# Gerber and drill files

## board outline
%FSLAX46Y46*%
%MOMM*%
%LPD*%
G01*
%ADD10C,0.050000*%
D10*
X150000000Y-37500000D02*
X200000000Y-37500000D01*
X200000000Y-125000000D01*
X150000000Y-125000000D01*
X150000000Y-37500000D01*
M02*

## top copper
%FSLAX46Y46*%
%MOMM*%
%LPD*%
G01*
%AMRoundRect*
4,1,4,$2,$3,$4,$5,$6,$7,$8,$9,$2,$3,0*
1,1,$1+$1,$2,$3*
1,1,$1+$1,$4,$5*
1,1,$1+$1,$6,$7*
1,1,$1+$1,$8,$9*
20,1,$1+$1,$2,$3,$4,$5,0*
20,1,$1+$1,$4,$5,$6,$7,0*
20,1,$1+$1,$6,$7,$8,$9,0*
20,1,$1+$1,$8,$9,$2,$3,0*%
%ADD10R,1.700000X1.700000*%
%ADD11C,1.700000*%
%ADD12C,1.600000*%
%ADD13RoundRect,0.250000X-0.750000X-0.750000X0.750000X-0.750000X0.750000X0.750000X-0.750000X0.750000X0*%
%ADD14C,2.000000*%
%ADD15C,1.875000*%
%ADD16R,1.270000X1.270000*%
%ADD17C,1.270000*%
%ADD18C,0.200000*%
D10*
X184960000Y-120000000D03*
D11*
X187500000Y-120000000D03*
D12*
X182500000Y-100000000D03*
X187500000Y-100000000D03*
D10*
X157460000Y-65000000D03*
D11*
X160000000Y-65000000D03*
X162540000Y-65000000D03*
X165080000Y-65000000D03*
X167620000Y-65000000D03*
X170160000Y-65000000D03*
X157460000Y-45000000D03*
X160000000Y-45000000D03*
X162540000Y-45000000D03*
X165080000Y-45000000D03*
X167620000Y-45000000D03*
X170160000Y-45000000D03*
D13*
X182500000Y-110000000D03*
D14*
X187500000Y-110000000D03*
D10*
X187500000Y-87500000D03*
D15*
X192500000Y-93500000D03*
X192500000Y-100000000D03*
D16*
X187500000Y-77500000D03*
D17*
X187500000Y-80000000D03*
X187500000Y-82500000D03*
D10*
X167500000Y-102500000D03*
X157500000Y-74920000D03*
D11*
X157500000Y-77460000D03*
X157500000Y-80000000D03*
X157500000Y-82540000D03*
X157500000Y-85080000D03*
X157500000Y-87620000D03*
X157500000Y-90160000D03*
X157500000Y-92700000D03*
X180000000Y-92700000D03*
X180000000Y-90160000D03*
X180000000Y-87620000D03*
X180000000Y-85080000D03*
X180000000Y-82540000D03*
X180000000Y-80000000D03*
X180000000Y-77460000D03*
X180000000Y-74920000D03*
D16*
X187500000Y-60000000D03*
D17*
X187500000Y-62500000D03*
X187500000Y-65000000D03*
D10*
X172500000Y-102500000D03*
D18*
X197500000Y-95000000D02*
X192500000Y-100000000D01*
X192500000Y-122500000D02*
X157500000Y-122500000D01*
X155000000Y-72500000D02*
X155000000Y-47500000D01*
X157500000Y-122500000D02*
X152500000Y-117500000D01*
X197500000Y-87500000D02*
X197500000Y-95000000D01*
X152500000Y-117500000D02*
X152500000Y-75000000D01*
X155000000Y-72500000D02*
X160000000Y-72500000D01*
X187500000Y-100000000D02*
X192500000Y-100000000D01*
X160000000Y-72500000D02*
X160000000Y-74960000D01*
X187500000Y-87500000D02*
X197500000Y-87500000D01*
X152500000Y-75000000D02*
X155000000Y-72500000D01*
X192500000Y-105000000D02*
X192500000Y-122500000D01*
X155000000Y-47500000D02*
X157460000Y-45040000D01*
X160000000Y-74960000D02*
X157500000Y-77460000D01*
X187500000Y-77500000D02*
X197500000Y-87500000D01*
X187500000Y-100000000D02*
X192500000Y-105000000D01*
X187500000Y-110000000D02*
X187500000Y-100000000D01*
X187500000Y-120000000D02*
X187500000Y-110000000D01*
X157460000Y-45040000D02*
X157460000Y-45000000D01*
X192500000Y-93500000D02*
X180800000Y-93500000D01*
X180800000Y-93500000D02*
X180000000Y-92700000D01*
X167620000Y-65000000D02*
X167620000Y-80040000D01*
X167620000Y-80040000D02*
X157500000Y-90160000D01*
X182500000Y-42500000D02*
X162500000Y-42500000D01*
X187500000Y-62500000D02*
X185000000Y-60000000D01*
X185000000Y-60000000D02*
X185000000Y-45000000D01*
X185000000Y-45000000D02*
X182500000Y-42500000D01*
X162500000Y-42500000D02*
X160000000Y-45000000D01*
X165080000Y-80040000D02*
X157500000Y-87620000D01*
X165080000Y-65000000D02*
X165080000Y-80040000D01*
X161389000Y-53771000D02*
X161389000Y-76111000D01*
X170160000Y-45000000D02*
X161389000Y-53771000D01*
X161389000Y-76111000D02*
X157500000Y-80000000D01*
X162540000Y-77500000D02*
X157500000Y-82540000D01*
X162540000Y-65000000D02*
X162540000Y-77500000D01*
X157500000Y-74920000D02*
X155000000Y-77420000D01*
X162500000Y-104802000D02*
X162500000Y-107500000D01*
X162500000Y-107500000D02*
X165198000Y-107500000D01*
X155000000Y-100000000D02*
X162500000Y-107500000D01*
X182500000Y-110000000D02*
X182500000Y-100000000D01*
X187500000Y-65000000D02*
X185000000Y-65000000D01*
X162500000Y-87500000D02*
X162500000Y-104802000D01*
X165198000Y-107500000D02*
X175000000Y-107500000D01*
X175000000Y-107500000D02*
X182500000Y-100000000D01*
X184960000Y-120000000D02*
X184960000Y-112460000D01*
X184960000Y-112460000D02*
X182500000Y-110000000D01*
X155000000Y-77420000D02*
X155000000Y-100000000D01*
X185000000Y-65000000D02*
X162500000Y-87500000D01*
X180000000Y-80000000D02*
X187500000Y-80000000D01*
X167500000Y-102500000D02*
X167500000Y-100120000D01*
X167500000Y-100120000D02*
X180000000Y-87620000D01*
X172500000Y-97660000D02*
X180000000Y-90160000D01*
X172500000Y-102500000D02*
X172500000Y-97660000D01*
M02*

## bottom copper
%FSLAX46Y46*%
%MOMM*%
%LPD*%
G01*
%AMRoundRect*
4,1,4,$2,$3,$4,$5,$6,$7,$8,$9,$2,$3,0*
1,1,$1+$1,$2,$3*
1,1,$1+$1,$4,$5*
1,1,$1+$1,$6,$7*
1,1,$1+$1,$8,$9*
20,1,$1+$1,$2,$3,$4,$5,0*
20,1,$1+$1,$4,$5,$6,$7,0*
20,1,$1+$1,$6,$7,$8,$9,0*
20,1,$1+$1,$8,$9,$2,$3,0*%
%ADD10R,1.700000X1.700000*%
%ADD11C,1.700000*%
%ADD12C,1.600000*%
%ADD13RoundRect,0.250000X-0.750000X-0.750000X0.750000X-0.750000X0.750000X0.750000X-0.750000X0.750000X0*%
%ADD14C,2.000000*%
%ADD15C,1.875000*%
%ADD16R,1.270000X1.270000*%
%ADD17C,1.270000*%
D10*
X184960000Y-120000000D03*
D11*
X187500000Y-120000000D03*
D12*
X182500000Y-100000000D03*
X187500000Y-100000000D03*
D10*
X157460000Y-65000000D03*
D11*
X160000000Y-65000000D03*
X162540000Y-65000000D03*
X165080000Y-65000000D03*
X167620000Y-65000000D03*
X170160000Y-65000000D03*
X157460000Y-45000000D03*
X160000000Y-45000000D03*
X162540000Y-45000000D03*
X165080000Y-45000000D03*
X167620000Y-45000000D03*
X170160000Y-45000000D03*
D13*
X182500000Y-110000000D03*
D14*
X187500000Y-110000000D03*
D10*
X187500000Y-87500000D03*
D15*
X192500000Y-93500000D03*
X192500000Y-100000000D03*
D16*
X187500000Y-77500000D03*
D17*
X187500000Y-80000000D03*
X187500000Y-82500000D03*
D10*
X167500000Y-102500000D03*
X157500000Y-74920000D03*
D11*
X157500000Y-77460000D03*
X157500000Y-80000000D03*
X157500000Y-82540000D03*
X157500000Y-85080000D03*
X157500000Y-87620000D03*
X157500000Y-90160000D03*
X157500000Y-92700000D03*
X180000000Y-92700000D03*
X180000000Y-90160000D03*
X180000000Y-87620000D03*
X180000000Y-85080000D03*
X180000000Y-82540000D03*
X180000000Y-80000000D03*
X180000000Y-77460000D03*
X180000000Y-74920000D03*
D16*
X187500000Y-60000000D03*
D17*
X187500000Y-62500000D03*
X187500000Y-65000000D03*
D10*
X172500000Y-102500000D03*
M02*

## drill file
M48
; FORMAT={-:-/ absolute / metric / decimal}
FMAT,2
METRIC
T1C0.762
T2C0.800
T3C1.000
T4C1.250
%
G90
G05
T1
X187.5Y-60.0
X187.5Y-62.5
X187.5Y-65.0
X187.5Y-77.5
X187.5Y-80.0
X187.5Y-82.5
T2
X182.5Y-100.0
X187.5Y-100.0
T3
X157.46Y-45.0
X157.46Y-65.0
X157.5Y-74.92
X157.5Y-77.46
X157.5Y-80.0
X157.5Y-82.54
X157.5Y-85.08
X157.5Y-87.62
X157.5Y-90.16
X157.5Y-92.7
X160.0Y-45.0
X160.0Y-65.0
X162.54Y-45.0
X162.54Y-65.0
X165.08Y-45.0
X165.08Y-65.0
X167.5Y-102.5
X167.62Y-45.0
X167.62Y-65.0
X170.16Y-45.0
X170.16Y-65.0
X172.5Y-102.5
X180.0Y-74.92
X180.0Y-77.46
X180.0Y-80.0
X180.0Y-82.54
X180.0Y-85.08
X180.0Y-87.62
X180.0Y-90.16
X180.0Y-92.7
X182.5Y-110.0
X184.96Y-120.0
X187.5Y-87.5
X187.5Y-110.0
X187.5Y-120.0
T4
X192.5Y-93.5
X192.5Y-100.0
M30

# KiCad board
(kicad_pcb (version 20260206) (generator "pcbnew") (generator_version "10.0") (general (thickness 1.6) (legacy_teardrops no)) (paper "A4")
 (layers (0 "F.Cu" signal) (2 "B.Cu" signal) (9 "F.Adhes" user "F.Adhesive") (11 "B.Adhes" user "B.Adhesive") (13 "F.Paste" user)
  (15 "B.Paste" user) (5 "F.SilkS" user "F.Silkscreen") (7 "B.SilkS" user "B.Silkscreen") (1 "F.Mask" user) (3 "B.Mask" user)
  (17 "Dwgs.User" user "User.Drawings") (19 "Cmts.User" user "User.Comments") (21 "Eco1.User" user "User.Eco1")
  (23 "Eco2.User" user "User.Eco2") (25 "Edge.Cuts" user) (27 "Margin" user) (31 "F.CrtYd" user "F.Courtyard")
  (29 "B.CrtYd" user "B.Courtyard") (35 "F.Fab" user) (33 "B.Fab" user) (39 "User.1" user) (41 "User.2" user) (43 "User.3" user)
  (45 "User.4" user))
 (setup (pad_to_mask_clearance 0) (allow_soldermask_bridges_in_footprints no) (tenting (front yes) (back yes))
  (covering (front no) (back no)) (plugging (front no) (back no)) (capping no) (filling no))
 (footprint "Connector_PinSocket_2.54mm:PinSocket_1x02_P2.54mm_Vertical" (layer "F.Cu") (at 184.96 120 90)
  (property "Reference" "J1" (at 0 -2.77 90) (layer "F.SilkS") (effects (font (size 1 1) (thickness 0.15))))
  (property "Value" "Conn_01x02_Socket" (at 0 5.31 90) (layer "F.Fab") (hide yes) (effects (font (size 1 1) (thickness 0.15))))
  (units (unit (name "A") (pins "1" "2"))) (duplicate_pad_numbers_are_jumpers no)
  (pad "1" thru_hole rect (at 0 0 90) (size 1.7 1.7) (drill 1) (layers "*.Cu" "*.Mask") (remove_unused_layers no) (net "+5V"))
  (pad "2" thru_hole circle (at 0 2.54 90) (size 1.7 1.7) (drill 1) (layers "*.Cu" "*.Mask") (remove_unused_layers no) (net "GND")))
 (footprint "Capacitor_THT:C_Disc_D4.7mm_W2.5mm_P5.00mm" (layer "F.Cu") (at 182.5 100)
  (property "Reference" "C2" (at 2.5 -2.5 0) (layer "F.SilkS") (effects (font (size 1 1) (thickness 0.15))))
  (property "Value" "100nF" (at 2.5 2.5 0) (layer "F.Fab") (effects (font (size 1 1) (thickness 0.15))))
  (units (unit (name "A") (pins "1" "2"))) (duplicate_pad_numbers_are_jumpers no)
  (pad "1" thru_hole circle (at 0 0) (size 1.6 1.6) (drill 0.8) (layers "*.Cu" "*.Mask") (remove_unused_layers no) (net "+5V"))
  (pad "2" thru_hole circle (at 5 0) (size 1.6 1.6) (drill 0.8) (layers "*.Cu" "*.Mask") (remove_unused_layers no) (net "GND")))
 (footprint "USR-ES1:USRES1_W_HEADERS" (layer "F.Cu") (at 163.69 55 90)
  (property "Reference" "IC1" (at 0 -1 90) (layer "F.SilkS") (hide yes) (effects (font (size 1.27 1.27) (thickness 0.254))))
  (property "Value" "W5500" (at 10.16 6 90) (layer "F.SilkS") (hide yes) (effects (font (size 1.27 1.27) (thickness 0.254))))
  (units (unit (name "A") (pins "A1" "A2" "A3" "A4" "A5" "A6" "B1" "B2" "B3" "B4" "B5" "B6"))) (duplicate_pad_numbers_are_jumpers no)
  (pad "A1" thru_hole rect (at -10 -6.23 90) (size 1.7 1.7) (drill 1) (layers "*.Cu" "*.Mask") (remove_unused_layers no)
   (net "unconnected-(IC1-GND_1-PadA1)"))
  (pad "A2" thru_hole circle (at -10 -3.69 90) (size 1.7 1.7) (drill 1) (layers "*.Cu" "*.Mask") (remove_unused_layers no)
   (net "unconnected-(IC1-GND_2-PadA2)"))
  (pad "A3" thru_hole circle (at -10 -1.15 90) (size 1.7 1.7) (drill 1) (layers "*.Cu" "*.Mask") (remove_unused_layers no)
   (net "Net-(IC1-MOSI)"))
  (pad "A4" thru_hole circle (at -10 1.39 90) (size 1.7 1.7) (drill 1) (layers "*.Cu" "*.Mask") (remove_unused_layers no)
   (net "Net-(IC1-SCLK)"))
  (pad "A5" thru_hole circle (at -10 3.93 90) (size 1.7 1.7) (drill 1) (layers "*.Cu" "*.Mask") (remove_unused_layers no)
   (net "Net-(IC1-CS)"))
  (pad "A6" thru_hole circle (at -10 6.47 90) (size 1.7 1.7) (drill 1) (layers "*.Cu" "*.Mask") (remove_unused_layers no)
   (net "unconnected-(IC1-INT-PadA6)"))
  (pad "B1" thru_hole circle (at 10 -6.23 90) (size 1.7 1.7) (drill 1) (layers "*.Cu" "*.Mask") (remove_unused_layers no) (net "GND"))
  (pad "B2" thru_hole circle (at 10 -3.69 90) (size 1.7 1.7) (drill 1) (layers "*.Cu" "*.Mask") (remove_unused_layers no)
   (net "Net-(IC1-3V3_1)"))
  (pad "B3" thru_hole circle (at 10 -1.15 90) (size 1.7 1.7) (drill 1) (layers "*.Cu" "*.Mask") (remove_unused_layers no)
   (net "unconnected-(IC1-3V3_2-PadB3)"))
  (pad "B4" thru_hole circle (at 10 1.39 90) (size 1.7 1.7) (drill 1) (layers "*.Cu" "*.Mask") (remove_unused_layers no)
   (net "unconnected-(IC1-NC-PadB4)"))
  (pad "B5" thru_hole circle (at 10 3.93 90) (size 1.7 1.7) (drill 1) (layers "*.Cu" "*.Mask") (remove_unused_layers no)
   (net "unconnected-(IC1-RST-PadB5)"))
  (pad "B6" thru_hole circle (at 10 6.47 90) (size 1.7 1.7) (drill 1) (layers "*.Cu" "*.Mask") (remove_unused_layers no)
   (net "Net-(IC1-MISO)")))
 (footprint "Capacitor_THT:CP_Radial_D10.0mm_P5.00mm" (layer "F.Cu") (at 182.5 110)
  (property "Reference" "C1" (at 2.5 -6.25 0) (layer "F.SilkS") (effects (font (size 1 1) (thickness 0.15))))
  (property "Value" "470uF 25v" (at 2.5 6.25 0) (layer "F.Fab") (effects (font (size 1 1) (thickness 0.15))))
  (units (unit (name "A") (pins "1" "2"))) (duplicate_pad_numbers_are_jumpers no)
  (pad "1" thru_hole roundrect (at 0 0) (size 2 2) (drill 1) (layers "*.Cu" "*.Mask") (remove_unused_layers no) (roundrect_rratio 0.125)
   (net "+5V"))
  (pad "2" thru_hole circle (at 5 0) (size 2 2) (drill 1) (layers "*.Cu" "*.Mask") (remove_unused_layers no) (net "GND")))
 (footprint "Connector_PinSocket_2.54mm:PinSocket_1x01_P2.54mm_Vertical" (layer "F.Cu") (at 187.5 87.5)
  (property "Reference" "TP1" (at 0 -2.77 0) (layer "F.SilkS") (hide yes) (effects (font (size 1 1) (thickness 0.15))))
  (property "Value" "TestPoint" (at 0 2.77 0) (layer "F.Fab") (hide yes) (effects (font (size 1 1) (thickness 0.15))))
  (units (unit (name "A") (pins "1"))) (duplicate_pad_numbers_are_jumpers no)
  (pad "1" thru_hole rect (at 0 0) (size 1.7 1.7) (drill 1) (layers "*.Cu" "*.Mask") (remove_unused_layers no) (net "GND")))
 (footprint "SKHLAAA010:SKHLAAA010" (layer "F.Cu") (at 192.5 96.75 -90)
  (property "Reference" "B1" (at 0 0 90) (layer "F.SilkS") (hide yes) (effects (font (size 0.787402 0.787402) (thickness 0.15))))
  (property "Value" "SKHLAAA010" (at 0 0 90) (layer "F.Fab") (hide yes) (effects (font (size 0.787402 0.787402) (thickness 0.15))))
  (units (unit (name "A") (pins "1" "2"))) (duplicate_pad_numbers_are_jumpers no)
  (pad "1" thru_hole circle (at -3.25 0 270) (size 1.875 1.875) (drill 1.25) (layers "*.Cu" "*.Mask") (remove_unused_layers no)
   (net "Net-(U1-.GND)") (solder_mask_margin 0.102))
  (pad "2" thru_hole circle (at 3.25 0 270) (size 1.875 1.875) (drill 1.25) (layers "*.Cu" "*.Mask") (remove_unused_layers no) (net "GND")
   (solder_mask_margin 0.102)))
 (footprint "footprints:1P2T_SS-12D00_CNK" (layer "F.Cu") (at 187.5 77.5)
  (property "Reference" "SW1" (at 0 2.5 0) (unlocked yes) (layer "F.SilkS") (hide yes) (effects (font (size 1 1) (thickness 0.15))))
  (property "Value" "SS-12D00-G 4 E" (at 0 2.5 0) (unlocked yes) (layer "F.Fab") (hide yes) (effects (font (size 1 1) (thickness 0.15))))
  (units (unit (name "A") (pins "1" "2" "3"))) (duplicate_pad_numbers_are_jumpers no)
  (pad "1" thru_hole rect (at 0 0) (size 1.27 1.27) (drill 0.762) (layers "*.Cu" "*.Mask") (remove_unused_layers no) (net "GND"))
  (pad "2" thru_hole circle (at 0 2.5) (size 1.27 1.27) (drill 0.762) (layers "*.Cu" "*.Mask") (remove_unused_layers no)
   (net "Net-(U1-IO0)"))
  (pad "3" thru_hole circle (at 0 5) (size 1.27 1.27) (drill 0.762) (layers "*.Cu" "*.Mask") (remove_unused_layers no)
   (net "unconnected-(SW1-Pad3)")))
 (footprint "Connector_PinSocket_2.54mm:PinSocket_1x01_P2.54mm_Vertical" (layer "F.Cu") (at 167.5 102.5)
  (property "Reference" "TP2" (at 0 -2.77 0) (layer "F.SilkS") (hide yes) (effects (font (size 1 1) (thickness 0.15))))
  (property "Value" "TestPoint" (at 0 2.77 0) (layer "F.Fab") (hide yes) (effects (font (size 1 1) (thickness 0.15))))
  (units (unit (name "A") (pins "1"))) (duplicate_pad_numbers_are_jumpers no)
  (pad "1" thru_hole rect (at 0 0) (size 1.7 1.7) (drill 1) (layers "*.Cu" "*.Mask") (remove_unused_layers no) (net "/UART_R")))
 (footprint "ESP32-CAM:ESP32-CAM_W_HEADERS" (layer "F.Cu") (at 168.73 83.7)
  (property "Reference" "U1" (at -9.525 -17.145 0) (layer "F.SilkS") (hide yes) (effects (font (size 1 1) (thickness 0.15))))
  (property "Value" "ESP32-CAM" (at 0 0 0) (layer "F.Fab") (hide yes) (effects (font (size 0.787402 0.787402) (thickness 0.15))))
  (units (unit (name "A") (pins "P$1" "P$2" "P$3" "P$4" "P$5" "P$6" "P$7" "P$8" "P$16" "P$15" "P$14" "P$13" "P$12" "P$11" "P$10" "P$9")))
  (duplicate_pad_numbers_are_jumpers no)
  (pad "P$1" thru_hole rect (at -11.23 -8.78) (size 1.7 1.7) (drill 1) (layers "*.Cu" "*.Mask") (remove_unused_layers no) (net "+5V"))
  (pad "P$2" thru_hole circle (at -11.23 -6.24) (size 1.7 1.7) (drill 1) (layers "*.Cu" "*.Mask") (remove_unused_layers no) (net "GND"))
  (pad "P$3" thru_hole circle (at -11.23 -3.7) (size 1.7 1.7) (drill 1) (layers "*.Cu" "*.Mask") (remove_unused_layers no)
   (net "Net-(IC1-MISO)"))
  (pad "P$4" thru_hole circle (at -11.23 -1.16) (size 1.7 1.7) (drill 1) (layers "*.Cu" "*.Mask") (remove_unused_layers no)
   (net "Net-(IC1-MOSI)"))
  (pad "P$5" thru_hole circle (at -11.23 1.38) (size 1.7 1.7) (drill 1) (layers "*.Cu" "*.Mask") (remove_unused_layers no)
   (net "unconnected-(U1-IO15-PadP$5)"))
  (pad "P$6" thru_hole circle (at -11.23 3.92) (size 1.7 1.7) (drill 1) (layers "*.Cu" "*.Mask") (remove_unused_layers no)
   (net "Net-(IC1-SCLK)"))
  (pad "P$7" thru_hole circle (at -11.23 6.46) (size 1.7 1.7) (drill 1) (layers "*.Cu" "*.Mask") (remove_unused_layers no)
   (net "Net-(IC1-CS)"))
  (pad "P$8" thru_hole circle (at -11.23 9) (size 1.7 1.7) (drill 1) (layers "*.Cu" "*.Mask") (remove_unused_layers no)
   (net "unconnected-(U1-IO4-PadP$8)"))
  (pad "P$9" thru_hole circle (at 11.27 9) (size 1.7 1.7) (drill 1) (layers "*.Cu" "*.Mask") (remove_unused_layers no) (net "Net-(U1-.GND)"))
  (pad "P$10" thru_hole circle (at 11.27 6.46) (size 1.7 1.7) (drill 1) (layers "*.Cu" "*.Mask") (remove_unused_layers no) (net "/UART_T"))
  (pad "P$11" thru_hole circle (at 11.27 3.92) (size 1.7 1.7) (drill 1) (layers "*.Cu" "*.Mask") (remove_unused_layers no) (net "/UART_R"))
  (pad "P$12" thru_hole circle (at 11.27 1.38) (size 1.7 1.7) (drill 1) (layers "*.Cu" "*.Mask") (remove_unused_layers no)
   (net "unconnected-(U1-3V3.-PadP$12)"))
  (pad "P$13" thru_hole circle (at 11.27 -1.16) (size 1.7 1.7) (drill 1) (layers "*.Cu" "*.Mask") (remove_unused_layers no)
   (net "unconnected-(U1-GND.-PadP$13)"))
  (pad "P$14" thru_hole circle (at 11.27 -3.7) (size 1.7 1.7) (drill 1) (layers "*.Cu" "*.Mask") (remove_unused_layers no)
   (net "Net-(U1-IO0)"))
  (pad "P$15" thru_hole circle (at 11.27 -6.24) (size 1.7 1.7) (drill 1) (layers "*.Cu" "*.Mask") (remove_unused_layers no)
   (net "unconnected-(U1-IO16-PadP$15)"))
  (pad "P$16" thru_hole circle (at 11.27 -8.78) (size 1.7 1.7) (drill 1) (layers "*.Cu" "*.Mask") (remove_unused_layers no)
   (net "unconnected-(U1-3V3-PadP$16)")))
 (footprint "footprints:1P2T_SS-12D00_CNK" (layer "F.Cu") (at 187.5 60)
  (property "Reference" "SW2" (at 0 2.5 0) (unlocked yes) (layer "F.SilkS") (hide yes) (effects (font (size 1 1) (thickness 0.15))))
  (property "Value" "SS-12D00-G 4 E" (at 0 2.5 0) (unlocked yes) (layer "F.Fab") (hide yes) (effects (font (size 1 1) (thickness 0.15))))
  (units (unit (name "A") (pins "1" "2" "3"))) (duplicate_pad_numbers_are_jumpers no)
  (pad "1" thru_hole rect (at 0 0) (size 1.27 1.27) (drill 0.762) (layers "*.Cu" "*.Mask") (remove_unused_layers no)
   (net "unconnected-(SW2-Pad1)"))
  (pad "2" thru_hole circle (at 0 2.5) (size 1.27 1.27) (drill 0.762) (layers "*.Cu" "*.Mask") (remove_unused_layers no)
   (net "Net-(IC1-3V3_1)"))
  (pad "3" thru_hole circle (at 0 5) (size 1.27 1.27) (drill 0.762) (layers "*.Cu" "*.Mask") (remove_unused_layers no) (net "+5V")))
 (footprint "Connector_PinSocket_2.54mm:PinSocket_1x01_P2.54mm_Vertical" (layer "F.Cu") (at 172.5 102.5)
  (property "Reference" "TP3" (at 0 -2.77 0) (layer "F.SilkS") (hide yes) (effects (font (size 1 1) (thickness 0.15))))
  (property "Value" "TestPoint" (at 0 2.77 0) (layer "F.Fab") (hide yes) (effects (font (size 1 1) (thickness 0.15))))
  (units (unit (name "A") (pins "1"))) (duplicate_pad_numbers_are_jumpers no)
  (pad "1" thru_hole rect (at 0 0) (size 1.7 1.7) (drill 1) (layers "*.Cu" "*.Mask") (remove_unused_layers no) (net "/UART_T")))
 (gr_rect (start 150 37.5) (end 200 125) (stroke (width 0.05) (type default)) (fill no) (layer "Edge.Cuts"))
 (segment (start 197.5 95) (end 192.5 100) (width 0.2) (layer "F.Cu") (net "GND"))
 (segment (start 192.5 122.5) (end 157.5 122.5) (width 0.2) (layer "F.Cu") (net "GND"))
 (segment (start 155 72.5) (end 155 47.5) (width 0.2) (layer "F.Cu") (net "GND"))
 (segment (start 157.5 122.5) (end 152.5 117.5) (width 0.2) (layer "F.Cu") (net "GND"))
 (segment (start 197.5 87.5) (end 197.5 95) (width 0.2) (layer "F.Cu") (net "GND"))
 (segment (start 152.5 117.5) (end 152.5 75) (width 0.2) (layer "F.Cu") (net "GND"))
 (segment (start 155 72.5) (end 160 72.5) (width 0.2) (layer "F.Cu") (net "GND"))
 (segment (start 187.5 100) (end 192.5 100) (width 0.2) (layer "F.Cu") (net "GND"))
 (segment (start 160 72.5) (end 160 74.96) (width 0.2) (layer "F.Cu") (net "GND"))
 (segment (start 187.5 87.5) (end 197.5 87.5) (width 0.2) (layer "F.Cu") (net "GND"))
 (segment (start 152.5 75) (end 155 72.5) (width 0.2) (layer "F.Cu") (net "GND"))
 (segment (start 192.5 105) (end 192.5 122.5) (width 0.2) (layer "F.Cu") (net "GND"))
 (segment (start 155 47.5) (end 157.46 45.04) (width 0.2) (layer "F.Cu") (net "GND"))
 (segment (start 160 74.96) (end 157.5 77.46) (width 0.2) (layer "F.Cu") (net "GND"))
 (segment (start 187.5 77.5) (end 197.5 87.5) (width 0.2) (layer "F.Cu") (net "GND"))
 (segment (start 187.5 100) (end 192.5 105) (width 0.2) (layer "F.Cu") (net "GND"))
 (segment (start 187.5 110) (end 187.5 100) (width 0.2) (layer "F.Cu") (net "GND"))
 (segment (start 187.5 120) (end 187.5 110) (width 0.2) (layer "F.Cu") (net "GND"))
 (segment (start 157.46 45.04) (end 157.46 45) (width 0.2) (layer "F.Cu") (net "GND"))
 (segment (start 192.5 93.5) (end 180.8 93.5) (width 0.2) (layer "F.Cu") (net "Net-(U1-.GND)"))
 (segment (start 180.8 93.5) (end 180 92.7) (width 0.2) (layer "F.Cu") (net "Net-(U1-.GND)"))
 (segment (start 167.62 65) (end 167.62 80.04) (width 0.2) (layer "F.Cu") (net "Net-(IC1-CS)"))
 (segment (start 167.62 80.04) (end 157.5 90.16) (width 0.2) (layer "F.Cu") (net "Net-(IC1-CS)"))
 (segment (start 182.5 42.5) (end 162.5 42.5) (width 0.2) (layer "F.Cu") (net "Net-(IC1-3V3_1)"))
 (segment (start 187.5 62.5) (end 185 60) (width 0.2) (layer "F.Cu") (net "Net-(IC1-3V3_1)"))
 (segment (start 185 60) (end 185 45) (width 0.2) (layer "F.Cu") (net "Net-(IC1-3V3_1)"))
 (segment (start 185 45) (end 182.5 42.5) (width 0.2) (layer "F.Cu") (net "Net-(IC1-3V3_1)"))
 (segment (start 162.5 42.5) (end 160 45) (width 0.2) (layer "F.Cu") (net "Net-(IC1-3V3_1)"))
 (segment (start 165.08 80.04) (end 157.5 87.62) (width 0.2) (layer "F.Cu") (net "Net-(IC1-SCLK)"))
 (segment (start 165.08 65) (end 165.08 80.04) (width 0.2) (layer "F.Cu") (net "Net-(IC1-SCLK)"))
 (segment (start 161.389 53.771) (end 161.389 76.111) (width 0.2) (layer "F.Cu") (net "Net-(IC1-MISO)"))
 (segment (start 170.16 45) (end 161.389 53.771) (width 0.2) (layer "F.Cu") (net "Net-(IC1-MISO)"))
 (segment (start 161.389 76.111) (end 157.5 80) (width 0.2) (layer "F.Cu") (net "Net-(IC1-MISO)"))
 (segment (start 162.54 77.5) (end 157.5 82.54) (width 0.2) (layer "F.Cu") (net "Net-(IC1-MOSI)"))
 (segment (start 162.54 65) (end 162.54 77.5) (width 0.2) (layer "F.Cu") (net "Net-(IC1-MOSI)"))
 (segment (start 157.5 74.92) (end 155 77.42) (width 0.2) (layer "F.Cu") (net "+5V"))
 (segment (start 162.5 104.802) (end 162.5 107.5) (width 0.2) (layer "F.Cu") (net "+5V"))
 (segment (start 162.5 107.5) (end 165.198 107.5) (width 0.2) (layer "F.Cu") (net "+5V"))
 (segment (start 155 100) (end 162.5 107.5) (width 0.2) (layer "F.Cu") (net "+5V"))
 (segment (start 182.5 110) (end 182.5 100) (width 0.2) (layer "F.Cu") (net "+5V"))
 (segment (start 187.5 65) (end 185 65) (width 0.2) (layer "F.Cu") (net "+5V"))
 (segment (start 162.5 87.5) (end 162.5 104.802) (width 0.2) (layer "F.Cu") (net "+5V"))
 (segment (start 165.198 107.5) (end 175 107.5) (width 0.2) (layer "F.Cu") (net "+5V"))
 (segment (start 175 107.5) (end 182.5 100) (width 0.2) (layer "F.Cu") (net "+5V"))
 (segment (start 184.96 120) (end 184.96 112.46) (width 0.2) (layer "F.Cu") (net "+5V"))
 (segment (start 184.96 112.46) (end 182.5 110) (width 0.2) (layer "F.Cu") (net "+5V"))
 (segment (start 155 77.42) (end 155 100) (width 0.2) (layer "F.Cu") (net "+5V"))
 (segment (start 185 65) (end 162.5 87.5) (width 0.2) (layer "F.Cu") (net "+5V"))
 (segment (start 180 80) (end 187.5 80) (width 0.2) (layer "F.Cu") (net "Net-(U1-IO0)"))
 (segment (start 167.5 102.5) (end 167.5 100.12) (width 0.2) (layer "F.Cu") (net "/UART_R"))
 (segment (start 167.5 100.12) (end 180 87.62) (width 0.2) (layer "F.Cu") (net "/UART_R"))
 (segment (start 172.5 97.66) (end 180 90.16) (width 0.2) (layer "F.Cu") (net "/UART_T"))
 (segment (start 172.5 102.5) (end 172.5 97.66) (width 0.2) (layer "F.Cu") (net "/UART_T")))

